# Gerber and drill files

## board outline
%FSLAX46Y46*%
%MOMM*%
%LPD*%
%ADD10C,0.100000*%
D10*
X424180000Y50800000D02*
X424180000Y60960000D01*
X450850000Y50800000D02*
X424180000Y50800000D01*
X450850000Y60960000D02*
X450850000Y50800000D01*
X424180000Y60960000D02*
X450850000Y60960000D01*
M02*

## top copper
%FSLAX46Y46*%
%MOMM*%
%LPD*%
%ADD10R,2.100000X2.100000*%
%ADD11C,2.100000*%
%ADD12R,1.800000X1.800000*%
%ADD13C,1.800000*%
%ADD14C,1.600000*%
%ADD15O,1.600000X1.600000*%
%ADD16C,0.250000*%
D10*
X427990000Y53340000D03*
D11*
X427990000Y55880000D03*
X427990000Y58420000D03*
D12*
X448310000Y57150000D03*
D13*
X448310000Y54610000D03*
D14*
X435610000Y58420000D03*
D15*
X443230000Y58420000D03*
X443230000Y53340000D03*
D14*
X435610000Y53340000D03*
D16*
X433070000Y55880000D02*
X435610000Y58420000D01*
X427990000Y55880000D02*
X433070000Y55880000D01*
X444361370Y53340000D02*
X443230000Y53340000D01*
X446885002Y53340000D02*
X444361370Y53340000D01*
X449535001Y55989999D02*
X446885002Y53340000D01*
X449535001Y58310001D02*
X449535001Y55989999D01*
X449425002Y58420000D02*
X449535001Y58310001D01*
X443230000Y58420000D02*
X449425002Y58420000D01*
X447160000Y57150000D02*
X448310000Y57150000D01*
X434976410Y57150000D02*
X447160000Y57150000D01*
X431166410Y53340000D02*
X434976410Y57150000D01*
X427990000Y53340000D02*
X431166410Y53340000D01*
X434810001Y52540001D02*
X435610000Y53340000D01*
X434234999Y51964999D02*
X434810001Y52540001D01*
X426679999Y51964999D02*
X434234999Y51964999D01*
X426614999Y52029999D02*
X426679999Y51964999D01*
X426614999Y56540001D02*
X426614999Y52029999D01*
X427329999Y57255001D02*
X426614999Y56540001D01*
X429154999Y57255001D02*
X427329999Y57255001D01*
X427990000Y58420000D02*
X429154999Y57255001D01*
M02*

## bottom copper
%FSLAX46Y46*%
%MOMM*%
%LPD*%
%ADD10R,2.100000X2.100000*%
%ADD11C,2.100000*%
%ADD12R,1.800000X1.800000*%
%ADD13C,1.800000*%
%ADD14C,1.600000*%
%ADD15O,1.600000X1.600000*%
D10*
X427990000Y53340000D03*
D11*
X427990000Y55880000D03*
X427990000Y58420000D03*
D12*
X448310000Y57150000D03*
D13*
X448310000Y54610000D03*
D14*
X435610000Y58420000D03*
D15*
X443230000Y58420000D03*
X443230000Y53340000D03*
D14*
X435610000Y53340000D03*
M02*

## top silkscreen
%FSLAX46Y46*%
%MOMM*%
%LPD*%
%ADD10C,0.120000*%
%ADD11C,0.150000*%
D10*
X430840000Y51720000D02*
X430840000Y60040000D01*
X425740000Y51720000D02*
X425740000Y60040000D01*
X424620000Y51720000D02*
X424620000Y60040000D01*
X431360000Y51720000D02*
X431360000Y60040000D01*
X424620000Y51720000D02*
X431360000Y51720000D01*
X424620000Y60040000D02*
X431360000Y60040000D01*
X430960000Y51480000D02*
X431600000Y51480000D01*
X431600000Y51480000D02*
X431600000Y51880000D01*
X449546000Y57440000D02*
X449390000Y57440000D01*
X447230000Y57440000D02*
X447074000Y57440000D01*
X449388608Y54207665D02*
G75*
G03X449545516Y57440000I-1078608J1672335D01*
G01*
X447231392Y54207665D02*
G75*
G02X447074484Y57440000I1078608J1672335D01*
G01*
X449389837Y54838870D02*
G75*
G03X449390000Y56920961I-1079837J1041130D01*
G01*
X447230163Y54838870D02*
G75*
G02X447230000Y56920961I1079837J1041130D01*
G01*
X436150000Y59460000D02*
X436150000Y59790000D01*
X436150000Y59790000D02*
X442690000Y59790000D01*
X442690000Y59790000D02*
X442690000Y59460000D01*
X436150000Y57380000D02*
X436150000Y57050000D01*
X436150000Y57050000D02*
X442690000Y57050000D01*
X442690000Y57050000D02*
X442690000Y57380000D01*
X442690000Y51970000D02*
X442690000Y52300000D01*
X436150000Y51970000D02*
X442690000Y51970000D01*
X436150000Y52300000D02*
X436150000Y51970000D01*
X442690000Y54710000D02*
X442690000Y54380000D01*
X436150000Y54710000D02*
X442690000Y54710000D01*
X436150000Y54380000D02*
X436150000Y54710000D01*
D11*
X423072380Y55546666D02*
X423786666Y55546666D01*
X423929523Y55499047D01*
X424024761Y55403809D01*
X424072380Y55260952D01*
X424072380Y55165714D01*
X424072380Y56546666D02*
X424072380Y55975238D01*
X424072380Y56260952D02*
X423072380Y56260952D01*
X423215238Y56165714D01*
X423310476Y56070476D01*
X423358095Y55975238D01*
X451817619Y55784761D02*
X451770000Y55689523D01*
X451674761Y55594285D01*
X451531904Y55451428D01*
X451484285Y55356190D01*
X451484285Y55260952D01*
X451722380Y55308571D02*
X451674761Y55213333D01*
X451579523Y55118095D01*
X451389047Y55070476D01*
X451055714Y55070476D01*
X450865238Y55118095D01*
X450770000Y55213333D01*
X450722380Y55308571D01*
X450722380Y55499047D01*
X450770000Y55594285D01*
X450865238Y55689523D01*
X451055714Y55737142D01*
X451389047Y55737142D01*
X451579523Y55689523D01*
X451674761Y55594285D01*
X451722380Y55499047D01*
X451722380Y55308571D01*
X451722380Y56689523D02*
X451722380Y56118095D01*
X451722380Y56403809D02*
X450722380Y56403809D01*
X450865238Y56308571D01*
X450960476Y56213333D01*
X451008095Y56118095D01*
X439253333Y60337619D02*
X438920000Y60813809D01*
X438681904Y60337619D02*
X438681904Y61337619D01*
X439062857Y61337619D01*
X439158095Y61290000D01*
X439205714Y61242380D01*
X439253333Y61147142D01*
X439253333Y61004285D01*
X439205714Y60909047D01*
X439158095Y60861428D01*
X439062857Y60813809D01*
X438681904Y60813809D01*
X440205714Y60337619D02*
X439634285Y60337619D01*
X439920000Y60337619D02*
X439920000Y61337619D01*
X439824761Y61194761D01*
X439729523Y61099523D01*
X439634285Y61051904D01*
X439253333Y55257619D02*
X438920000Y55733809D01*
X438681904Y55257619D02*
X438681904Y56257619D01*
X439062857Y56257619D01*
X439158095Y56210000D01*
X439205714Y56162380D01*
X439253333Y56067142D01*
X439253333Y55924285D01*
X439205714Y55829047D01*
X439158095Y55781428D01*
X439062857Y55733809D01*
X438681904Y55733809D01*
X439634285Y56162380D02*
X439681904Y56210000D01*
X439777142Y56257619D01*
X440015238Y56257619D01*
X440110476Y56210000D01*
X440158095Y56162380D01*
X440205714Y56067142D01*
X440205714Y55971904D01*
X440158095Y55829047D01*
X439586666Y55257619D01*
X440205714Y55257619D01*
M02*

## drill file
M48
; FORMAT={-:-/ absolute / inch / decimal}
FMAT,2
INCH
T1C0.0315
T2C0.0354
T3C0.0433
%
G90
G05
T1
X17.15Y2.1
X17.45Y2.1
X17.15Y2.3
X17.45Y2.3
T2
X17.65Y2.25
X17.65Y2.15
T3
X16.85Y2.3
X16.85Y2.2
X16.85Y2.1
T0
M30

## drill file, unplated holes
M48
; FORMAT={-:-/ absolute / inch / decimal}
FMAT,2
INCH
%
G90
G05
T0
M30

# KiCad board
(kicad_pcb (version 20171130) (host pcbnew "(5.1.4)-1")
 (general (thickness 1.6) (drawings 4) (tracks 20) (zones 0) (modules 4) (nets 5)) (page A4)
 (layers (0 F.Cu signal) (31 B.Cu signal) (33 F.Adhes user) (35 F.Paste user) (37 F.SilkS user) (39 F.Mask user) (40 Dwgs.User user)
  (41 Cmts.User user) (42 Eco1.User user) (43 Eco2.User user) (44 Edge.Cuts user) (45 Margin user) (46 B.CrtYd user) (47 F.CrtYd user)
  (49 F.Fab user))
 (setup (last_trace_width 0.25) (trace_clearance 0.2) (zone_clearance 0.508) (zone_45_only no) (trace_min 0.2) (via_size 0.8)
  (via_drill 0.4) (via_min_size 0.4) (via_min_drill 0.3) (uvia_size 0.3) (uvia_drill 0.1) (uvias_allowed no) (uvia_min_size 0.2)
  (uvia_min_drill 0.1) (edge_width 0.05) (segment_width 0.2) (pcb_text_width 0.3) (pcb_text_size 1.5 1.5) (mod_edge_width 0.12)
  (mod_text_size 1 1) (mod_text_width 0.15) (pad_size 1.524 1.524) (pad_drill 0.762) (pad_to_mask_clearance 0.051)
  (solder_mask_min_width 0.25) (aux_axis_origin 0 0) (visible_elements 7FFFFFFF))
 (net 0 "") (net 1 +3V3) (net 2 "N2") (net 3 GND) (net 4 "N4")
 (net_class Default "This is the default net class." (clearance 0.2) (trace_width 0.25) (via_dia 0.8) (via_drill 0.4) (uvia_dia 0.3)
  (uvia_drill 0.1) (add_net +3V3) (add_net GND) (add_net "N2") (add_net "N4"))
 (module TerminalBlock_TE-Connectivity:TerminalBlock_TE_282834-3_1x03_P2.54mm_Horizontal (layer F.Cu) (at 427.99 -53.34 90)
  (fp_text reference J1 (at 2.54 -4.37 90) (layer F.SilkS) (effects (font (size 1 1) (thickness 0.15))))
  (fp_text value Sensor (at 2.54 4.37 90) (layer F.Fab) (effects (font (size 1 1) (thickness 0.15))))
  (fp_line (start -1.62 2.85) (end 6.7 2.85) (layer F.SilkS) (width 0.12))
  (fp_line (start -1.62 -2.25) (end 6.7 -2.25) (layer F.SilkS) (width 0.12))
  (fp_line (start -1.62 -3.37) (end 6.7 -3.37) (layer F.SilkS) (width 0.12))
  (fp_line (start -1.62 3.37) (end 6.7 3.37) (layer F.SilkS) (width 0.12))
  (fp_line (start -1.62 -3.37) (end -1.62 3.37) (layer F.SilkS) (width 0.12))
  (fp_line (start 6.7 -3.37) (end 6.7 3.37) (layer F.SilkS) (width 0.12))
  (fp_line (start -1.86 2.97) (end -1.86 3.61) (layer F.SilkS) (width 0.12))
  (fp_line (start -1.86 3.61) (end -1.46 3.61) (layer F.SilkS) (width 0.12))
  (pad 1 thru_hole rect (at 0 0 90) (size 2.1 2.1) (drill 1.1) (layers *.Cu *.Mask) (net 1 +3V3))
  (pad 2 thru_hole circle (at 2.54 0 90) (size 2.1 2.1) (drill 1.1) (layers *.Cu *.Mask) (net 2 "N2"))
  (pad 3 thru_hole circle (at 5.08 0 90) (size 2.1 2.1) (drill 1.1) (layers *.Cu *.Mask) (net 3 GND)))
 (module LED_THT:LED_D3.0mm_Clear (layer F.Cu) (at 448.31 -57.15 270)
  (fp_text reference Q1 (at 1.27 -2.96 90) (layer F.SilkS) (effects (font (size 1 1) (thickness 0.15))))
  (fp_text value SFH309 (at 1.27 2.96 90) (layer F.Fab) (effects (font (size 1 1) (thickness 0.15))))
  (fp_line (start -0.29 -1.236) (end -0.29 -1.08) (layer F.SilkS) (width 0.12))
  (fp_line (start -0.29 1.08) (end -0.29 1.236) (layer F.SilkS) (width 0.12))
  (fp_arc (start 1.27 0) (end -0.29 -1.235516) (angle 108.8) (layer F.SilkS) (width 0.12))
  (fp_arc (start 1.27 0) (end -0.29 1.235516) (angle -108.8) (layer F.SilkS) (width 0.12))
  (fp_arc (start 1.27 0) (end 0.229039 -1.08) (angle 87.9) (layer F.SilkS) (width 0.12))
  (fp_arc (start 1.27 0) (end 0.229039 1.08) (angle -87.9) (layer F.SilkS) (width 0.12))
  (pad 1 thru_hole rect (at 0 0 270) (size 1.8 1.8) (drill 0.9) (layers *.Cu *.Mask) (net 1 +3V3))
  (pad 2 thru_hole circle (at 2.54 0 270) (size 1.8 1.8) (drill 0.9) (layers *.Cu *.Mask) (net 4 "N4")))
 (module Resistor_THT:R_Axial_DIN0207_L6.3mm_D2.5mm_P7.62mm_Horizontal (layer F.Cu) (at 435.61 -58.42)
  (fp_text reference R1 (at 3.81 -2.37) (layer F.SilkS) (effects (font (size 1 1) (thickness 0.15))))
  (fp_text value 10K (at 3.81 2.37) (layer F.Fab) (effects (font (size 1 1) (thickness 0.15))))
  (fp_line (start 0.54 -1.04) (end 0.54 -1.37) (layer F.SilkS) (width 0.12))
  (fp_line (start 0.54 -1.37) (end 7.08 -1.37) (layer F.SilkS) (width 0.12))
  (fp_line (start 7.08 -1.37) (end 7.08 -1.04) (layer F.SilkS) (width 0.12))
  (fp_line (start 0.54 1.04) (end 0.54 1.37) (layer F.SilkS) (width 0.12))
  (fp_line (start 0.54 1.37) (end 7.08 1.37) (layer F.SilkS) (width 0.12))
  (fp_line (start 7.08 1.37) (end 7.08 1.04) (layer F.SilkS) (width 0.12))
  (pad 1 thru_hole circle (at 0 0) (size 1.6 1.6) (drill 0.8) (layers *.Cu *.Mask) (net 2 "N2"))
  (pad 2 thru_hole oval (at 7.62 0) (size 1.6 1.6) (drill 0.8) (layers *.Cu *.Mask) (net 4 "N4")))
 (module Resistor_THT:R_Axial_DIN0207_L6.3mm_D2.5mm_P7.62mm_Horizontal (layer F.Cu) (at 435.61 -53.34)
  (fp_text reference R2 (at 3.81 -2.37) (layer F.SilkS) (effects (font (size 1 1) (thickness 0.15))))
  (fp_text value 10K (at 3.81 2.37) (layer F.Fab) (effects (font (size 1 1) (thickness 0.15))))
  (fp_line (start 7.08 1.37) (end 7.08 1.04) (layer F.SilkS) (width 0.12))
  (fp_line (start 0.54 1.37) (end 7.08 1.37) (layer F.SilkS) (width 0.12))
  (fp_line (start 0.54 1.04) (end 0.54 1.37) (layer F.SilkS) (width 0.12))
  (fp_line (start 7.08 -1.37) (end 7.08 -1.04) (layer F.SilkS) (width 0.12))
  (fp_line (start 0.54 -1.37) (end 7.08 -1.37) (layer F.SilkS) (width 0.12))
  (fp_line (start 0.54 -1.04) (end 0.54 -1.37) (layer F.SilkS) (width 0.12))
  (pad 2 thru_hole oval (at 7.62 0) (size 1.6 1.6) (drill 0.8) (layers *.Cu *.Mask) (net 4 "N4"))
  (pad 1 thru_hole circle (at 0 0) (size 1.6 1.6) (drill 0.8) (layers *.Cu *.Mask) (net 3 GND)))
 (gr_line (start 424.18 -50.8) (end 424.18 -60.96) (layer Edge.Cuts) (width 0.1))
 (gr_line (start 450.85 -50.8) (end 424.18 -50.8) (layer Edge.Cuts) (width 0.1))
 (gr_line (start 450.85 -60.96) (end 450.85 -50.8) (layer Edge.Cuts) (width 0.1))
 (gr_line (start 424.18 -60.96) (end 450.85 -60.96) (layer Edge.Cuts) (width 0.1))
 (segment (start 433.07 -55.88) (end 435.61 -58.42) (width 0.25) (layer F.Cu) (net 2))
 (segment (start 427.99 -55.88) (end 433.07 -55.88) (width 0.25) (layer F.Cu) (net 2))
 (segment (start 444.36137 -53.34) (end 443.23 -53.34) (width 0.25) (layer F.Cu) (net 4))
 (segment (start 446.885002 -53.34) (end 444.36137 -53.34) (width 0.25) (layer F.Cu) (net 4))
 (segment (start 449.535001 -55.989999) (end 446.885002 -53.34) (width 0.25) (layer F.Cu) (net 4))
 (segment (start 449.535001 -58.310001) (end 449.535001 -55.989999) (width 0.25) (layer F.Cu) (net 4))
 (segment (start 449.425002 -58.42) (end 449.535001 -58.310001) (width 0.25) (layer F.Cu) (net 4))
 (segment (start 443.23 -58.42) (end 449.425002 -58.42) (width 0.25) (layer F.Cu) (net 4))
 (segment (start 447.16 -57.15) (end 448.31 -57.15) (width 0.25) (layer F.Cu) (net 1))
 (segment (start 434.97641 -57.15) (end 447.16 -57.15) (width 0.25) (layer F.Cu) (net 1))
 (segment (start 431.16641 -53.34) (end 434.97641 -57.15) (width 0.25) (layer F.Cu) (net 1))
 (segment (start 427.99 -53.34) (end 431.16641 -53.34) (width 0.25) (layer F.Cu) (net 1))
 (segment (start 434.810001 -52.540001) (end 435.61 -53.34) (width 0.25) (layer F.Cu) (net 3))
 (segment (start 434.234999 -51.964999) (end 434.810001 -52.540001) (width 0.25) (layer F.Cu) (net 3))
 (segment (start 426.679999 -51.964999) (end 434.234999 -51.964999) (width 0.25) (layer F.Cu) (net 3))
 (segment (start 426.614999 -52.029999) (end 426.679999 -51.964999) (width 0.25) (layer F.Cu) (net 3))
 (segment (start 426.614999 -56.540001) (end 426.614999 -52.029999) (width 0.25) (layer F.Cu) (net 3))
 (segment (start 427.329999 -57.255001) (end 426.614999 -56.540001) (width 0.25) (layer F.Cu) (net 3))
 (segment (start 429.154999 -57.255001) (end 427.329999 -57.255001) (width 0.25) (layer F.Cu) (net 3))
 (segment (start 427.99 -58.42) (end 429.154999 -57.255001) (width 0.25) (layer F.Cu) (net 3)))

